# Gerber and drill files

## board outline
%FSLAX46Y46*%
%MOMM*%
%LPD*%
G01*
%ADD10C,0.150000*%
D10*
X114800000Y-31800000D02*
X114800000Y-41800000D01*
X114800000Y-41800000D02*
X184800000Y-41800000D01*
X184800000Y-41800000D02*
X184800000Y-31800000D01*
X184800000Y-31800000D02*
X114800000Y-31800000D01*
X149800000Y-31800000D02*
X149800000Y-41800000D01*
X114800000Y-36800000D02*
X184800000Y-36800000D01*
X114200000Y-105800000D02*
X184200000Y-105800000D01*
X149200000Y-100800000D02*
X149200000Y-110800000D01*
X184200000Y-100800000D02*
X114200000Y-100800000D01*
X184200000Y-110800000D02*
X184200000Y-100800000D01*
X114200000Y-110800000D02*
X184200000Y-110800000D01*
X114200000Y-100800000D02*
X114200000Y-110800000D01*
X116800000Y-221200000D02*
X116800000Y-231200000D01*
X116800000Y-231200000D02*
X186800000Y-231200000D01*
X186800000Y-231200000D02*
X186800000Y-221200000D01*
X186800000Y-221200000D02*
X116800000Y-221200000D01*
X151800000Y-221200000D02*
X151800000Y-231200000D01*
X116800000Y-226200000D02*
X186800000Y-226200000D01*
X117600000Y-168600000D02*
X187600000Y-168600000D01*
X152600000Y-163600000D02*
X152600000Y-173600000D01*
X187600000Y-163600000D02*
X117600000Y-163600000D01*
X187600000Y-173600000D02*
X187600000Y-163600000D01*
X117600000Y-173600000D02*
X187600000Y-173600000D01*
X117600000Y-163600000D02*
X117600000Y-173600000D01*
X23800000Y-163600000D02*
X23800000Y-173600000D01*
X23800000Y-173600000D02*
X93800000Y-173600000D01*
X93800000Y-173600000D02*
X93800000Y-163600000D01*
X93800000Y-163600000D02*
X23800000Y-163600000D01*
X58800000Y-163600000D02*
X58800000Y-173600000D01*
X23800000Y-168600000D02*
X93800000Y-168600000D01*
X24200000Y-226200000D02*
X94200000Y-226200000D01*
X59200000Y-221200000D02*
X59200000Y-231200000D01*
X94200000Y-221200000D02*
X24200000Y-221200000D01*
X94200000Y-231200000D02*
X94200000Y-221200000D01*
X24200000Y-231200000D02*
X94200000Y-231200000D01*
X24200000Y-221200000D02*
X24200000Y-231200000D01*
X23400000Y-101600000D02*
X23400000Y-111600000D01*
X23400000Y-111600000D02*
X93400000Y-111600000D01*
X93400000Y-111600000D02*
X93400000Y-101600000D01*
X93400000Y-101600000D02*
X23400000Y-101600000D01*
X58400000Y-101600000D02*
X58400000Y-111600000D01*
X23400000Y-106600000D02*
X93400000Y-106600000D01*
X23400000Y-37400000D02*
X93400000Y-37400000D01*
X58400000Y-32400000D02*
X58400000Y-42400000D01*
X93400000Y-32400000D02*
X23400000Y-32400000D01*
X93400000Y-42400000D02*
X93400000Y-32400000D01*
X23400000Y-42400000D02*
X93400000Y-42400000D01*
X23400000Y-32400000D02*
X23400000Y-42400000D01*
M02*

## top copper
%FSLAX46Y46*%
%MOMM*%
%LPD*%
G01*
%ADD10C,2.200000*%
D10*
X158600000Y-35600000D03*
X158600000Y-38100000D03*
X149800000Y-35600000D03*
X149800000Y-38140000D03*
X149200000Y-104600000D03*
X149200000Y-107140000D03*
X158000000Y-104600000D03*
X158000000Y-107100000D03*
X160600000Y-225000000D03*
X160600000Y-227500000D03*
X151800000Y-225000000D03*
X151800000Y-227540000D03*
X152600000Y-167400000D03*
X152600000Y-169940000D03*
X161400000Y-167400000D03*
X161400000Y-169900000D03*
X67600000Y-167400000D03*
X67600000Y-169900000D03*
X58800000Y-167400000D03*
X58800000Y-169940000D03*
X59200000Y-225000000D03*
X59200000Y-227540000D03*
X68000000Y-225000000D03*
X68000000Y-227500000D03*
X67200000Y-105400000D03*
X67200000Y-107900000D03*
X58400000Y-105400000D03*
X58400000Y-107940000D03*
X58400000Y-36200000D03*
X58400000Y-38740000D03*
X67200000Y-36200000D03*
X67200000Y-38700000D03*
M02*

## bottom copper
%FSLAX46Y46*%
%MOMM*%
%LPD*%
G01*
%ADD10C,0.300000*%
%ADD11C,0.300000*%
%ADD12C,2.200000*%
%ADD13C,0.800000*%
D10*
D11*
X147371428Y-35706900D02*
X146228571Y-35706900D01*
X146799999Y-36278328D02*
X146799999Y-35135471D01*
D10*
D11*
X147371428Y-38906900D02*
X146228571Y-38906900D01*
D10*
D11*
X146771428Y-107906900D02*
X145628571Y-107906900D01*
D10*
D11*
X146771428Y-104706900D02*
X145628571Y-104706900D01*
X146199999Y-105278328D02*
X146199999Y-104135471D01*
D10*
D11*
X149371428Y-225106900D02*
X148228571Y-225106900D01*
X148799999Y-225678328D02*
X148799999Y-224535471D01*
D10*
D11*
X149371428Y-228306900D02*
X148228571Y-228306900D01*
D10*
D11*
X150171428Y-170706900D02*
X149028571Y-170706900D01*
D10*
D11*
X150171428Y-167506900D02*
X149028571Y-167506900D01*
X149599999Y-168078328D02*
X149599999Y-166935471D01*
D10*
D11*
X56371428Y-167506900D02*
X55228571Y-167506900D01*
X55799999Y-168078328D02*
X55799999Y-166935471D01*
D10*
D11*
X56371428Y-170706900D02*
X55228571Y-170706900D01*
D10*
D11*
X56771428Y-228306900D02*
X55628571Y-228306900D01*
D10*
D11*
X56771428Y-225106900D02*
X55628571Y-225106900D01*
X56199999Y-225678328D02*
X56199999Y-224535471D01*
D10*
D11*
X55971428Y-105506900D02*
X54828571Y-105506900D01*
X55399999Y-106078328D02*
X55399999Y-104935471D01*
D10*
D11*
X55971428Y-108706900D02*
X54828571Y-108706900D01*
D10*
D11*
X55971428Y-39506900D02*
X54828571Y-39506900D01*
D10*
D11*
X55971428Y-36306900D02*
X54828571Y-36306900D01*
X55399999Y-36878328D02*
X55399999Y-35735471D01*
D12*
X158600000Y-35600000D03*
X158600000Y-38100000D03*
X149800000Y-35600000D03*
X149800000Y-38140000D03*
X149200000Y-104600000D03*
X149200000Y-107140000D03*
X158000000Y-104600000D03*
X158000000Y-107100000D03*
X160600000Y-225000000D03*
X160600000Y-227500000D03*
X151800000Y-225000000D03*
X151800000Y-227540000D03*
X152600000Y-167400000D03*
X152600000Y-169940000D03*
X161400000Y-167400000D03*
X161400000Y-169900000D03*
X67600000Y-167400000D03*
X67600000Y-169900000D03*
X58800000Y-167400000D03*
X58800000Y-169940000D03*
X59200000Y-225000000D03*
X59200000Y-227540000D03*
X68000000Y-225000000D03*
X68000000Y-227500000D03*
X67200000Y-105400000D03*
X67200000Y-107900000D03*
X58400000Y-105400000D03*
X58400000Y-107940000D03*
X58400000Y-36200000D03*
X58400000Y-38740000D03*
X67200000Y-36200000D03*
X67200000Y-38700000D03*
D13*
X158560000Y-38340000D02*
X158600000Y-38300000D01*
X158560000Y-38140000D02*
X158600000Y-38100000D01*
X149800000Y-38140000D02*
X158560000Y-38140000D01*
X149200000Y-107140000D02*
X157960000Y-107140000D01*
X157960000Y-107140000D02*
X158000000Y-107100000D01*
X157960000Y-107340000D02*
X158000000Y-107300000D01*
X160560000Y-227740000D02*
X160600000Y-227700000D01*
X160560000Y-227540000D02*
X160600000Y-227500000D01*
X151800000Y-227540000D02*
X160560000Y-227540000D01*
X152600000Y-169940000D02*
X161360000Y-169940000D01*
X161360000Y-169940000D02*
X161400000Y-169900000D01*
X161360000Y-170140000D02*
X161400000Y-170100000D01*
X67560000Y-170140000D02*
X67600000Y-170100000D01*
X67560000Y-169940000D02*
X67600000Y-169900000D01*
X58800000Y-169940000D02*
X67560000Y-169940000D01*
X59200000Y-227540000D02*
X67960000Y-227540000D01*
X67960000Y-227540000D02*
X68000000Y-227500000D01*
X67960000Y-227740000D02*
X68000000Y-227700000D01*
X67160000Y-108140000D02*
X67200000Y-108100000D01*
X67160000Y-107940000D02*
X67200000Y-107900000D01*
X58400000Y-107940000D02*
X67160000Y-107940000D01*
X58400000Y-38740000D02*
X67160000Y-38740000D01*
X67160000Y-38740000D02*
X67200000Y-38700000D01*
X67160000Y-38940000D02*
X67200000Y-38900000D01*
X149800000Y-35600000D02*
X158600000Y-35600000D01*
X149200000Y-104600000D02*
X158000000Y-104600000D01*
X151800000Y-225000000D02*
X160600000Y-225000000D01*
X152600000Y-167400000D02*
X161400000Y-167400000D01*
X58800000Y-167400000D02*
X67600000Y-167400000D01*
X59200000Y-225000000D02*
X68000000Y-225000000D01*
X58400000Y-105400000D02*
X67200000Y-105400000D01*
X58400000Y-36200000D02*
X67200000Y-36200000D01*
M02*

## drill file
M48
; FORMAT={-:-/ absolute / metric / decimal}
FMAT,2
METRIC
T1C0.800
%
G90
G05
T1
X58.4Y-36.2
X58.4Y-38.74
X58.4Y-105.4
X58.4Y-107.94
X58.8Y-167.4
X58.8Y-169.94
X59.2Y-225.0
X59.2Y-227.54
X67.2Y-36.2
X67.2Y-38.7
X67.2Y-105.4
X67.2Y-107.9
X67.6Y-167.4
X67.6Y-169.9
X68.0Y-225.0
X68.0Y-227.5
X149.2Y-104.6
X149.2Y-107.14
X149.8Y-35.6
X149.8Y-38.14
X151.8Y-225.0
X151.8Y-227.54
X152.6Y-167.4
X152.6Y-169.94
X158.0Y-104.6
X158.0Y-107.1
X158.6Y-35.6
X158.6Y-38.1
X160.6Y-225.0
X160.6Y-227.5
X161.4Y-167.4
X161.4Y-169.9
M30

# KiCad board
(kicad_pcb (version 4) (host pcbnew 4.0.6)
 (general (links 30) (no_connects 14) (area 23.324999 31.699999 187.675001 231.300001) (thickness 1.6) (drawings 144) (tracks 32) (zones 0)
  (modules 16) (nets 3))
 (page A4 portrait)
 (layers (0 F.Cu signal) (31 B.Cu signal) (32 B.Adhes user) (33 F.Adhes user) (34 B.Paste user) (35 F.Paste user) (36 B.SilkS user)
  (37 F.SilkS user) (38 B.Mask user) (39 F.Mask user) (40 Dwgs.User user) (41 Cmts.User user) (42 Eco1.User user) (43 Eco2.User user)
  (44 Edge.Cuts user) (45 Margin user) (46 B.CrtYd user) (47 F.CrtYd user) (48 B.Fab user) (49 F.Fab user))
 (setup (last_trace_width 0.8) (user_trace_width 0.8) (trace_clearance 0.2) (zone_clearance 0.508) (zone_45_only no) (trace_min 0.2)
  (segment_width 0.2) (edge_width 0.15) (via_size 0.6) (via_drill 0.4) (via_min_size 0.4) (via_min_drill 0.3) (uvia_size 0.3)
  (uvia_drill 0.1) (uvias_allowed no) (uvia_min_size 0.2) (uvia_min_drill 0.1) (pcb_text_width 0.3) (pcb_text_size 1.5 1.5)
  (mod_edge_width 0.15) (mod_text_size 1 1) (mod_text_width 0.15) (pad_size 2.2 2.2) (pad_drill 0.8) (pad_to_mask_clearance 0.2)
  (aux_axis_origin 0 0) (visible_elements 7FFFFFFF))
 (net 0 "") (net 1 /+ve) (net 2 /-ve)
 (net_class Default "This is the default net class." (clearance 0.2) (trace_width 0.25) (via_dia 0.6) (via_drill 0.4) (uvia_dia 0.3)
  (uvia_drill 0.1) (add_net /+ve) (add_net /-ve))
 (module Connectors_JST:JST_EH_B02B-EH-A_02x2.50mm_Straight (layer F.Cu) (at 158.6 35.6 270)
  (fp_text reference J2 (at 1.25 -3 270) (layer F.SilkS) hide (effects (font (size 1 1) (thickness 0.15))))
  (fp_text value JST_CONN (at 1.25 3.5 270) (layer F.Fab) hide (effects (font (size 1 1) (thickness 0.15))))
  (pad 1 thru_hole circle (at 0 0 270) (size 2.2 2.2) (drill 0.8) (layers *.Cu *.Mask) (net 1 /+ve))
  (pad 2 thru_hole circle (at 2.5 0 270) (size 2.2 2.2) (drill 0.8) (layers *.Cu *.Mask) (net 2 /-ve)))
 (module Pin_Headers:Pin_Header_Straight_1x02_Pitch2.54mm (layer F.Cu) (at 149.8 35.6)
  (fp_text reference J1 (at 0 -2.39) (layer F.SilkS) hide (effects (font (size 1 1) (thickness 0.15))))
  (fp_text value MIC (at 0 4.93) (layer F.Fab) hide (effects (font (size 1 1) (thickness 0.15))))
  (pad 1 thru_hole circle (at 0 0) (size 2.2 2.2) (drill 0.8) (layers *.Cu *.Mask) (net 1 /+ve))
  (pad 2 thru_hole circle (at 0 2.54) (size 2.2 2.2) (drill 0.8) (layers *.Cu *.Mask) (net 2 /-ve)))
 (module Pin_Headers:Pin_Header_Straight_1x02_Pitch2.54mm (layer F.Cu) (at 149.2 104.6)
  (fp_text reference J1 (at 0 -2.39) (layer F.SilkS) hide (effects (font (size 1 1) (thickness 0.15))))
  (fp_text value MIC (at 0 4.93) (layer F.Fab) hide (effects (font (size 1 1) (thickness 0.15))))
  (pad 1 thru_hole circle (at 0 0) (size 2.2 2.2) (drill 0.8) (layers *.Cu *.Mask) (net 1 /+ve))
  (pad 2 thru_hole circle (at 0 2.54) (size 2.2 2.2) (drill 0.8) (layers *.Cu *.Mask) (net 2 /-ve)))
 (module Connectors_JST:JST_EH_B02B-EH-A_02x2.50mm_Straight (layer F.Cu) (at 158 104.6 270)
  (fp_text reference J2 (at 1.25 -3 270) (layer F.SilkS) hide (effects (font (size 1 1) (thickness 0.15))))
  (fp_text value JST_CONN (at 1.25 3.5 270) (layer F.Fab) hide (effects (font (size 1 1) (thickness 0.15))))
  (pad 1 thru_hole circle (at 0 0 270) (size 2.2 2.2) (drill 0.8) (layers *.Cu *.Mask) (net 1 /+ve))
  (pad 2 thru_hole circle (at 2.5 0 270) (size 2.2 2.2) (drill 0.8) (layers *.Cu *.Mask) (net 2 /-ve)))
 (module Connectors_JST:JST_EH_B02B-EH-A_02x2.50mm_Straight (layer F.Cu) (at 160.6 225 270)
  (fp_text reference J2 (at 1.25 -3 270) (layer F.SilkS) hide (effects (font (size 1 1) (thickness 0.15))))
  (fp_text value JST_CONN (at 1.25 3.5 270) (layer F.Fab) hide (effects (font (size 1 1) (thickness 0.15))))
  (pad 1 thru_hole circle (at 0 0 270) (size 2.2 2.2) (drill 0.8) (layers *.Cu *.Mask) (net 1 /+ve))
  (pad 2 thru_hole circle (at 2.5 0 270) (size 2.2 2.2) (drill 0.8) (layers *.Cu *.Mask) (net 2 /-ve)))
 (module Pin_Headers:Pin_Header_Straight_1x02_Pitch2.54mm (layer F.Cu) (at 151.8 225)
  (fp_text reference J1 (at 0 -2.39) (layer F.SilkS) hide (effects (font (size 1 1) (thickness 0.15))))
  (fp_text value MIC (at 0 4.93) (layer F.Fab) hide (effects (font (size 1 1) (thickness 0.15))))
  (pad 1 thru_hole circle (at 0 0) (size 2.2 2.2) (drill 0.8) (layers *.Cu *.Mask) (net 1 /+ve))
  (pad 2 thru_hole circle (at 0 2.54) (size 2.2 2.2) (drill 0.8) (layers *.Cu *.Mask) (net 2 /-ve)))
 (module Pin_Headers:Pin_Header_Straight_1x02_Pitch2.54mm (layer F.Cu) (at 152.6 167.4)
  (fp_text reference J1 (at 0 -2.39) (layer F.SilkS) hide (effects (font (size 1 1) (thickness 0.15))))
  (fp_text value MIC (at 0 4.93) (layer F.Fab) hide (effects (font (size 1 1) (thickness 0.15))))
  (pad 1 thru_hole circle (at 0 0) (size 2.2 2.2) (drill 0.8) (layers *.Cu *.Mask) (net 1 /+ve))
  (pad 2 thru_hole circle (at 0 2.54) (size 2.2 2.2) (drill 0.8) (layers *.Cu *.Mask) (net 2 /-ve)))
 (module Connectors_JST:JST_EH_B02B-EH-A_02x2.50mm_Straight (layer F.Cu) (at 161.4 167.4 270)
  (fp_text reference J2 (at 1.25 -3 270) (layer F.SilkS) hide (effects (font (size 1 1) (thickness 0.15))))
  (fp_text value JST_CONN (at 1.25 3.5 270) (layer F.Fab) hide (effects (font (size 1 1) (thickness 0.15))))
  (pad 1 thru_hole circle (at 0 0 270) (size 2.2 2.2) (drill 0.8) (layers *.Cu *.Mask) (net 1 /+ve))
  (pad 2 thru_hole circle (at 2.5 0 270) (size 2.2 2.2) (drill 0.8) (layers *.Cu *.Mask) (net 2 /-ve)))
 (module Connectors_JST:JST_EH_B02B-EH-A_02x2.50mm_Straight (layer F.Cu) (at 67.6 167.4 270)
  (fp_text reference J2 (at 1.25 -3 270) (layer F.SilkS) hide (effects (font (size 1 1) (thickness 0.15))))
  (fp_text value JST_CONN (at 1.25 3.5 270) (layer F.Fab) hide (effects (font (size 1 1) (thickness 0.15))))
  (pad 1 thru_hole circle (at 0 0 270) (size 2.2 2.2) (drill 0.8) (layers *.Cu *.Mask) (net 1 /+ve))
  (pad 2 thru_hole circle (at 2.5 0 270) (size 2.2 2.2) (drill 0.8) (layers *.Cu *.Mask) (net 2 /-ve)))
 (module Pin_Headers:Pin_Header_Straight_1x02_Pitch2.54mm (layer F.Cu) (at 58.8 167.4)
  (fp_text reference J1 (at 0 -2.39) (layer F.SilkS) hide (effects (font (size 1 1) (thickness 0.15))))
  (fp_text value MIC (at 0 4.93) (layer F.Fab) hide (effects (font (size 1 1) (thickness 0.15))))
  (pad 1 thru_hole circle (at 0 0) (size 2.2 2.2) (drill 0.8) (layers *.Cu *.Mask) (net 1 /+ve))
  (pad 2 thru_hole circle (at 0 2.54) (size 2.2 2.2) (drill 0.8) (layers *.Cu *.Mask) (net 2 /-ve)))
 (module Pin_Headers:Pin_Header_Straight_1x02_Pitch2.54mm (layer F.Cu) (at 59.2 225)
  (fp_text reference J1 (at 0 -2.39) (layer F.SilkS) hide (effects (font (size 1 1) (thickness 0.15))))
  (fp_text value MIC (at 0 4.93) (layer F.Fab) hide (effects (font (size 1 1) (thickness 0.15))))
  (pad 1 thru_hole circle (at 0 0) (size 2.2 2.2) (drill 0.8) (layers *.Cu *.Mask) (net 1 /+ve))
  (pad 2 thru_hole circle (at 0 2.54) (size 2.2 2.2) (drill 0.8) (layers *.Cu *.Mask) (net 2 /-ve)))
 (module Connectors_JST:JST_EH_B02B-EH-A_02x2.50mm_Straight (layer F.Cu) (at 68 225 270)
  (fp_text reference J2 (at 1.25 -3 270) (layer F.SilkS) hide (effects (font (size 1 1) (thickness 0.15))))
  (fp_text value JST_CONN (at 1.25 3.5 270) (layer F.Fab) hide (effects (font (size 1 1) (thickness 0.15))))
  (pad 1 thru_hole circle (at 0 0 270) (size 2.2 2.2) (drill 0.8) (layers *.Cu *.Mask) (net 1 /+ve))
  (pad 2 thru_hole circle (at 2.5 0 270) (size 2.2 2.2) (drill 0.8) (layers *.Cu *.Mask) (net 2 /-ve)))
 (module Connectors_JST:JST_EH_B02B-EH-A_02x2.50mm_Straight (layer F.Cu) (at 67.2 105.4 270)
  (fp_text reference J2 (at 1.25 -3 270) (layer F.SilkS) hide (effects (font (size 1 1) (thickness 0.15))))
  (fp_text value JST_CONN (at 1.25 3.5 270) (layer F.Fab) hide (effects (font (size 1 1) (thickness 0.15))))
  (pad 1 thru_hole circle (at 0 0 270) (size 2.2 2.2) (drill 0.8) (layers *.Cu *.Mask) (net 1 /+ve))
  (pad 2 thru_hole circle (at 2.5 0 270) (size 2.2 2.2) (drill 0.8) (layers *.Cu *.Mask) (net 2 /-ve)))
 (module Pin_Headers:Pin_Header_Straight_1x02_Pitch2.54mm (layer F.Cu) (at 58.4 105.4)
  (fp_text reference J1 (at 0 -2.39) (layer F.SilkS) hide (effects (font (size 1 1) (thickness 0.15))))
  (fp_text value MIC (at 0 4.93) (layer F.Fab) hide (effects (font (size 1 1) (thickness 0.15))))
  (pad 1 thru_hole circle (at 0 0) (size 2.2 2.2) (drill 0.8) (layers *.Cu *.Mask) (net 1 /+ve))
  (pad 2 thru_hole circle (at 0 2.54) (size 2.2 2.2) (drill 0.8) (layers *.Cu *.Mask) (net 2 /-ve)))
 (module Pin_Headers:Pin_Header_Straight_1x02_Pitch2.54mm (layer F.Cu) (at 58.4 36.2)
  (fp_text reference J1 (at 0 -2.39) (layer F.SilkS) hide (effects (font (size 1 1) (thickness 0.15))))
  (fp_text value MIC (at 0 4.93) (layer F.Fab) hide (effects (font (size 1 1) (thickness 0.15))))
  (pad 1 thru_hole circle (at 0 0) (size 2.2 2.2) (drill 0.8) (layers *.Cu *.Mask) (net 1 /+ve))
  (pad 2 thru_hole circle (at 0 2.54) (size 2.2 2.2) (drill 0.8) (layers *.Cu *.Mask) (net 2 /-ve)))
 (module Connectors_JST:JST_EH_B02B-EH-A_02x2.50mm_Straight (layer F.Cu) (at 67.2 36.2 270)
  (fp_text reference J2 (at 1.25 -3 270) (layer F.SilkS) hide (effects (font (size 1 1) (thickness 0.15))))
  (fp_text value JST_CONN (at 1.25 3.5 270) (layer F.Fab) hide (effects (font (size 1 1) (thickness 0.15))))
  (pad 1 thru_hole circle (at 0 0 270) (size 2.2 2.2) (drill 0.8) (layers *.Cu *.Mask) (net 1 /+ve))
  (pad 2 thru_hole circle (at 2.5 0 270) (size 2.2 2.2) (drill 0.8) (layers *.Cu *.Mask) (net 2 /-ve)))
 (gr_line (start 114.8 31.8) (end 114.8 41.8) (angle 90) (layer Edge.Cuts) (width 0.15))
 (gr_line (start 114.8 41.8) (end 184.8 41.8) (angle 90) (layer Edge.Cuts) (width 0.15))
 (gr_line (start 184.8 41.8) (end 184.8 31.8) (angle 90) (layer Edge.Cuts) (width 0.15))
 (gr_line (start 184.8 31.8) (end 114.8 31.8) (angle 90) (layer Edge.Cuts) (width 0.15))
 (gr_line (start 149.8 31.8) (end 149.8 41.8) (angle 90) (layer Edge.Cuts) (width 0.15))
 (gr_line (start 114.8 36.8) (end 184.8 36.8) (angle 90) (layer Edge.Cuts) (width 0.15))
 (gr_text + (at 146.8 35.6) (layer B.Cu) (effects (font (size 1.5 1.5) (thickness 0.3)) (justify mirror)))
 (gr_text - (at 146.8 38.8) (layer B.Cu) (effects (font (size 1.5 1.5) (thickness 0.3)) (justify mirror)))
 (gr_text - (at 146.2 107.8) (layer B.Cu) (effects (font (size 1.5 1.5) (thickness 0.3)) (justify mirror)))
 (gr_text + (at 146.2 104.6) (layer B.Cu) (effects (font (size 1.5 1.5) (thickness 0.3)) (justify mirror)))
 (gr_line (start 114.2 105.8) (end 184.2 105.8) (angle 90) (layer Edge.Cuts) (width 0.15))
 (gr_line (start 149.2 100.8) (end 149.2 110.8) (angle 90) (layer Edge.Cuts) (width 0.15))
 (gr_line (start 184.2 100.8) (end 114.2 100.8) (angle 90) (layer Edge.Cuts) (width 0.15))
 (gr_line (start 184.2 110.8) (end 184.2 100.8) (angle 90) (layer Edge.Cuts) (width 0.15))
 (gr_line (start 114.2 110.8) (end 184.2 110.8) (angle 90) (layer Edge.Cuts) (width 0.15))
 (gr_line (start 114.2 100.8) (end 114.2 110.8) (angle 90) (layer Edge.Cuts) (width 0.15))
 (gr_line (start 116.8 221.2) (end 116.8 231.2) (angle 90) (layer Edge.Cuts) (width 0.15))
 (gr_line (start 116.8 231.2) (end 186.8 231.2) (angle 90) (layer Edge.Cuts) (width 0.15))
 (gr_line (start 186.8 231.2) (end 186.8 221.2) (angle 90) (layer Edge.Cuts) (width 0.15))
 (gr_line (start 186.8 221.2) (end 116.8 221.2) (angle 90) (layer Edge.Cuts) (width 0.15))
 (gr_line (start 151.8 221.2) (end 151.8 231.2) (angle 90) (layer Edge.Cuts) (width 0.15))
 (gr_line (start 116.8 226.2) (end 186.8 226.2) (angle 90) (layer Edge.Cuts) (width 0.15))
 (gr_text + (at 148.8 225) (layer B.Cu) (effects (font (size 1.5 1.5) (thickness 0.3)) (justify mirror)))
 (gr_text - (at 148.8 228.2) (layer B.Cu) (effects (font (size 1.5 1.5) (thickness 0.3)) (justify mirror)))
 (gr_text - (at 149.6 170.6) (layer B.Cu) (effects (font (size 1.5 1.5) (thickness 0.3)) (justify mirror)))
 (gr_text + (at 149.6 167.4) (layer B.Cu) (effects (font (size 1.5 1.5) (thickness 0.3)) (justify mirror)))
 (gr_line (start 117.6 168.6) (end 187.6 168.6) (angle 90) (layer Edge.Cuts) (width 0.15))
 (gr_line (start 152.6 163.6) (end 152.6 173.6) (angle 90) (layer Edge.Cuts) (width 0.15))
 (gr_line (start 187.6 163.6) (end 117.6 163.6) (angle 90) (layer Edge.Cuts) (width 0.15))
 (gr_line (start 187.6 173.6) (end 187.6 163.6) (angle 90) (layer Edge.Cuts) (width 0.15))
 (gr_line (start 117.6 173.6) (end 187.6 173.6) (angle 90) (layer Edge.Cuts) (width 0.15))
 (gr_line (start 117.6 163.6) (end 117.6 173.6) (angle 90) (layer Edge.Cuts) (width 0.15))
 (gr_line (start 23.8 163.6) (end 23.8 173.6) (angle 90) (layer Edge.Cuts) (width 0.15))
 (gr_line (start 23.8 173.6) (end 93.8 173.6) (angle 90) (layer Edge.Cuts) (width 0.15))
 (gr_line (start 93.8 173.6) (end 93.8 163.6) (angle 90) (layer Edge.Cuts) (width 0.15))
 (gr_line (start 93.8 163.6) (end 23.8 163.6) (angle 90) (layer Edge.Cuts) (width 0.15))
 (gr_line (start 58.8 163.6) (end 58.8 173.6) (angle 90) (layer Edge.Cuts) (width 0.15))
 (gr_line (start 23.8 168.6) (end 93.8 168.6) (angle 90) (layer Edge.Cuts) (width 0.15))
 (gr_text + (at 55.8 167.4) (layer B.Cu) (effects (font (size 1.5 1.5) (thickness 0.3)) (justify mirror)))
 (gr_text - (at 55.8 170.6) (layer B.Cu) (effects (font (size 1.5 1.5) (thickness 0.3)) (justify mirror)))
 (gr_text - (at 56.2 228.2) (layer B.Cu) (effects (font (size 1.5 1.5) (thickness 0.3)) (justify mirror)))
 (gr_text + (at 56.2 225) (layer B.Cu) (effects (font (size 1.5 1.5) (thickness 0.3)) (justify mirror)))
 (gr_line (start 24.2 226.2) (end 94.2 226.2) (angle 90) (layer Edge.Cuts) (width 0.15))
 (gr_line (start 59.2 221.2) (end 59.2 231.2) (angle 90) (layer Edge.Cuts) (width 0.15))
 (gr_line (start 94.2 221.2) (end 24.2 221.2) (angle 90) (layer Edge.Cuts) (width 0.15))
 (gr_line (start 94.2 231.2) (end 94.2 221.2) (angle 90) (layer Edge.Cuts) (width 0.15))
 (gr_line (start 24.2 231.2) (end 94.2 231.2) (angle 90) (layer Edge.Cuts) (width 0.15))
 (gr_line (start 24.2 221.2) (end 24.2 231.2) (angle 90) (layer Edge.Cuts) (width 0.15))
 (gr_line (start 23.4 101.6) (end 23.4 111.6) (angle 90) (layer Edge.Cuts) (width 0.15))
 (gr_line (start 23.4 111.6) (end 93.4 111.6) (angle 90) (layer Edge.Cuts) (width 0.15))
 (gr_line (start 93.4 111.6) (end 93.4 101.6) (angle 90) (layer Edge.Cuts) (width 0.15))
 (gr_line (start 93.4 101.6) (end 23.4 101.6) (angle 90) (layer Edge.Cuts) (width 0.15))
 (gr_line (start 58.4 101.6) (end 58.4 111.6) (angle 90) (layer Edge.Cuts) (width 0.15))
 (gr_line (start 23.4 106.6) (end 93.4 106.6) (angle 90) (layer Edge.Cuts) (width 0.15))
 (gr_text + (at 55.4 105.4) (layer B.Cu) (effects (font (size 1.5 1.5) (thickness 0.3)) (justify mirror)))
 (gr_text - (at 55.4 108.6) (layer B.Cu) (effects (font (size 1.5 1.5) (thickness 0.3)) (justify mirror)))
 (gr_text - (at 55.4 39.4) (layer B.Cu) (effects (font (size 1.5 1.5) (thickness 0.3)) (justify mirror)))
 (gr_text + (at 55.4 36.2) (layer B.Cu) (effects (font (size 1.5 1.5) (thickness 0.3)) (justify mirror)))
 (gr_line (start 23.4 37.4) (end 93.4 37.4) (angle 90) (layer Edge.Cuts) (width 0.15))
 (gr_line (start 58.4 32.4) (end 58.4 42.4) (angle 90) (layer Edge.Cuts) (width 0.15))
 (gr_line (start 93.4 32.4) (end 23.4 32.4) (angle 90) (layer Edge.Cuts) (width 0.15))
 (gr_line (start 93.4 42.4) (end 93.4 32.4) (angle 90) (layer Edge.Cuts) (width 0.15))
 (gr_line (start 23.4 42.4) (end 93.4 42.4) (angle 90) (layer Edge.Cuts) (width 0.15))
 (gr_line (start 23.4 32.4) (end 23.4 42.4) (angle 90) (layer Edge.Cuts) (width 0.15))
 (segment (start 158.56 38.34) (end 158.6 38.3) (width 0.8) (layer B.Cu) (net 2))
 (segment (start 158.56 38.14) (end 158.6 38.1) (width 0.8) (layer B.Cu) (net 2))
 (segment (start 149.8 38.14) (end 158.56 38.14) (width 0.8) (layer B.Cu) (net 2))
 (segment (start 149.2 107.14) (end 157.96 107.14) (width 0.8) (layer B.Cu) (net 2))
 (segment (start 157.96 107.14) (end 158 107.1) (width 0.8) (layer B.Cu) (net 2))
 (segment (start 157.96 107.34) (end 158 107.3) (width 0.8) (layer B.Cu) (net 2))
 (segment (start 160.56 227.74) (end 160.6 227.7) (width 0.8) (layer B.Cu) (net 2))
 (segment (start 160.56 227.54) (end 160.6 227.5) (width 0.8) (layer B.Cu) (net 2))
 (segment (start 151.8 227.54) (end 160.56 227.54) (width 0.8) (layer B.Cu) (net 2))
 (segment (start 152.6 169.94) (end 161.36 169.94) (width 0.8) (layer B.Cu) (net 2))
 (segment (start 161.36 169.94) (end 161.4 169.9) (width 0.8) (layer B.Cu) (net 2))
 (segment (start 161.36 170.14) (end 161.4 170.1) (width 0.8) (layer B.Cu) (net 2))
 (segment (start 67.56 170.14) (end 67.6 170.1) (width 0.8) (layer B.Cu) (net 2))
 (segment (start 67.56 169.94) (end 67.6 169.9) (width 0.8) (layer B.Cu) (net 2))
 (segment (start 58.8 169.94) (end 67.56 169.94) (width 0.8) (layer B.Cu) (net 2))
 (segment (start 59.2 227.54) (end 67.96 227.54) (width 0.8) (layer B.Cu) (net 2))
 (segment (start 67.96 227.54) (end 68 227.5) (width 0.8) (layer B.Cu) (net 2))
 (segment (start 67.96 227.74) (end 68 227.7) (width 0.8) (layer B.Cu) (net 2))
 (segment (start 67.16 108.14) (end 67.2 108.1) (width 0.8) (layer B.Cu) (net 2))
 (segment (start 67.16 107.94) (end 67.2 107.9) (width 0.8) (layer B.Cu) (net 2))
 (segment (start 58.4 107.94) (end 67.16 107.94) (width 0.8) (layer B.Cu) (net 2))
 (segment (start 58.4 38.74) (end 67.16 38.74) (width 0.8) (layer B.Cu) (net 2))
 (segment (start 67.16 38.74) (end 67.2 38.7) (width 0.8) (layer B.Cu) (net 2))
 (segment (start 67.16 38.94) (end 67.2 38.9) (width 0.8) (layer B.Cu) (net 2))
 (segment (start 149.8 35.6) (end 158.6 35.6) (width 0.8) (layer B.Cu) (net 1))
 (segment (start 149.2 104.6) (end 158 104.6) (width 0.8) (layer B.Cu) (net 1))
 (segment (start 151.8 225) (end 160.6 225) (width 0.8) (layer B.Cu) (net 1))
 (segment (start 152.6 167.4) (end 161.4 167.4) (width 0.8) (layer B.Cu) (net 1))
 (segment (start 58.8 167.4) (end 67.6 167.4) (width 0.8) (layer B.Cu) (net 1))
 (segment (start 59.2 225) (end 68 225) (width 0.8) (layer B.Cu) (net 1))
 (segment (start 58.4 105.4) (end 67.2 105.4) (width 0.8) (layer B.Cu) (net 1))
 (segment (start 58.4 36.2) (end 67.2 36.2) (width 0.8) (layer B.Cu) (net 1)))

